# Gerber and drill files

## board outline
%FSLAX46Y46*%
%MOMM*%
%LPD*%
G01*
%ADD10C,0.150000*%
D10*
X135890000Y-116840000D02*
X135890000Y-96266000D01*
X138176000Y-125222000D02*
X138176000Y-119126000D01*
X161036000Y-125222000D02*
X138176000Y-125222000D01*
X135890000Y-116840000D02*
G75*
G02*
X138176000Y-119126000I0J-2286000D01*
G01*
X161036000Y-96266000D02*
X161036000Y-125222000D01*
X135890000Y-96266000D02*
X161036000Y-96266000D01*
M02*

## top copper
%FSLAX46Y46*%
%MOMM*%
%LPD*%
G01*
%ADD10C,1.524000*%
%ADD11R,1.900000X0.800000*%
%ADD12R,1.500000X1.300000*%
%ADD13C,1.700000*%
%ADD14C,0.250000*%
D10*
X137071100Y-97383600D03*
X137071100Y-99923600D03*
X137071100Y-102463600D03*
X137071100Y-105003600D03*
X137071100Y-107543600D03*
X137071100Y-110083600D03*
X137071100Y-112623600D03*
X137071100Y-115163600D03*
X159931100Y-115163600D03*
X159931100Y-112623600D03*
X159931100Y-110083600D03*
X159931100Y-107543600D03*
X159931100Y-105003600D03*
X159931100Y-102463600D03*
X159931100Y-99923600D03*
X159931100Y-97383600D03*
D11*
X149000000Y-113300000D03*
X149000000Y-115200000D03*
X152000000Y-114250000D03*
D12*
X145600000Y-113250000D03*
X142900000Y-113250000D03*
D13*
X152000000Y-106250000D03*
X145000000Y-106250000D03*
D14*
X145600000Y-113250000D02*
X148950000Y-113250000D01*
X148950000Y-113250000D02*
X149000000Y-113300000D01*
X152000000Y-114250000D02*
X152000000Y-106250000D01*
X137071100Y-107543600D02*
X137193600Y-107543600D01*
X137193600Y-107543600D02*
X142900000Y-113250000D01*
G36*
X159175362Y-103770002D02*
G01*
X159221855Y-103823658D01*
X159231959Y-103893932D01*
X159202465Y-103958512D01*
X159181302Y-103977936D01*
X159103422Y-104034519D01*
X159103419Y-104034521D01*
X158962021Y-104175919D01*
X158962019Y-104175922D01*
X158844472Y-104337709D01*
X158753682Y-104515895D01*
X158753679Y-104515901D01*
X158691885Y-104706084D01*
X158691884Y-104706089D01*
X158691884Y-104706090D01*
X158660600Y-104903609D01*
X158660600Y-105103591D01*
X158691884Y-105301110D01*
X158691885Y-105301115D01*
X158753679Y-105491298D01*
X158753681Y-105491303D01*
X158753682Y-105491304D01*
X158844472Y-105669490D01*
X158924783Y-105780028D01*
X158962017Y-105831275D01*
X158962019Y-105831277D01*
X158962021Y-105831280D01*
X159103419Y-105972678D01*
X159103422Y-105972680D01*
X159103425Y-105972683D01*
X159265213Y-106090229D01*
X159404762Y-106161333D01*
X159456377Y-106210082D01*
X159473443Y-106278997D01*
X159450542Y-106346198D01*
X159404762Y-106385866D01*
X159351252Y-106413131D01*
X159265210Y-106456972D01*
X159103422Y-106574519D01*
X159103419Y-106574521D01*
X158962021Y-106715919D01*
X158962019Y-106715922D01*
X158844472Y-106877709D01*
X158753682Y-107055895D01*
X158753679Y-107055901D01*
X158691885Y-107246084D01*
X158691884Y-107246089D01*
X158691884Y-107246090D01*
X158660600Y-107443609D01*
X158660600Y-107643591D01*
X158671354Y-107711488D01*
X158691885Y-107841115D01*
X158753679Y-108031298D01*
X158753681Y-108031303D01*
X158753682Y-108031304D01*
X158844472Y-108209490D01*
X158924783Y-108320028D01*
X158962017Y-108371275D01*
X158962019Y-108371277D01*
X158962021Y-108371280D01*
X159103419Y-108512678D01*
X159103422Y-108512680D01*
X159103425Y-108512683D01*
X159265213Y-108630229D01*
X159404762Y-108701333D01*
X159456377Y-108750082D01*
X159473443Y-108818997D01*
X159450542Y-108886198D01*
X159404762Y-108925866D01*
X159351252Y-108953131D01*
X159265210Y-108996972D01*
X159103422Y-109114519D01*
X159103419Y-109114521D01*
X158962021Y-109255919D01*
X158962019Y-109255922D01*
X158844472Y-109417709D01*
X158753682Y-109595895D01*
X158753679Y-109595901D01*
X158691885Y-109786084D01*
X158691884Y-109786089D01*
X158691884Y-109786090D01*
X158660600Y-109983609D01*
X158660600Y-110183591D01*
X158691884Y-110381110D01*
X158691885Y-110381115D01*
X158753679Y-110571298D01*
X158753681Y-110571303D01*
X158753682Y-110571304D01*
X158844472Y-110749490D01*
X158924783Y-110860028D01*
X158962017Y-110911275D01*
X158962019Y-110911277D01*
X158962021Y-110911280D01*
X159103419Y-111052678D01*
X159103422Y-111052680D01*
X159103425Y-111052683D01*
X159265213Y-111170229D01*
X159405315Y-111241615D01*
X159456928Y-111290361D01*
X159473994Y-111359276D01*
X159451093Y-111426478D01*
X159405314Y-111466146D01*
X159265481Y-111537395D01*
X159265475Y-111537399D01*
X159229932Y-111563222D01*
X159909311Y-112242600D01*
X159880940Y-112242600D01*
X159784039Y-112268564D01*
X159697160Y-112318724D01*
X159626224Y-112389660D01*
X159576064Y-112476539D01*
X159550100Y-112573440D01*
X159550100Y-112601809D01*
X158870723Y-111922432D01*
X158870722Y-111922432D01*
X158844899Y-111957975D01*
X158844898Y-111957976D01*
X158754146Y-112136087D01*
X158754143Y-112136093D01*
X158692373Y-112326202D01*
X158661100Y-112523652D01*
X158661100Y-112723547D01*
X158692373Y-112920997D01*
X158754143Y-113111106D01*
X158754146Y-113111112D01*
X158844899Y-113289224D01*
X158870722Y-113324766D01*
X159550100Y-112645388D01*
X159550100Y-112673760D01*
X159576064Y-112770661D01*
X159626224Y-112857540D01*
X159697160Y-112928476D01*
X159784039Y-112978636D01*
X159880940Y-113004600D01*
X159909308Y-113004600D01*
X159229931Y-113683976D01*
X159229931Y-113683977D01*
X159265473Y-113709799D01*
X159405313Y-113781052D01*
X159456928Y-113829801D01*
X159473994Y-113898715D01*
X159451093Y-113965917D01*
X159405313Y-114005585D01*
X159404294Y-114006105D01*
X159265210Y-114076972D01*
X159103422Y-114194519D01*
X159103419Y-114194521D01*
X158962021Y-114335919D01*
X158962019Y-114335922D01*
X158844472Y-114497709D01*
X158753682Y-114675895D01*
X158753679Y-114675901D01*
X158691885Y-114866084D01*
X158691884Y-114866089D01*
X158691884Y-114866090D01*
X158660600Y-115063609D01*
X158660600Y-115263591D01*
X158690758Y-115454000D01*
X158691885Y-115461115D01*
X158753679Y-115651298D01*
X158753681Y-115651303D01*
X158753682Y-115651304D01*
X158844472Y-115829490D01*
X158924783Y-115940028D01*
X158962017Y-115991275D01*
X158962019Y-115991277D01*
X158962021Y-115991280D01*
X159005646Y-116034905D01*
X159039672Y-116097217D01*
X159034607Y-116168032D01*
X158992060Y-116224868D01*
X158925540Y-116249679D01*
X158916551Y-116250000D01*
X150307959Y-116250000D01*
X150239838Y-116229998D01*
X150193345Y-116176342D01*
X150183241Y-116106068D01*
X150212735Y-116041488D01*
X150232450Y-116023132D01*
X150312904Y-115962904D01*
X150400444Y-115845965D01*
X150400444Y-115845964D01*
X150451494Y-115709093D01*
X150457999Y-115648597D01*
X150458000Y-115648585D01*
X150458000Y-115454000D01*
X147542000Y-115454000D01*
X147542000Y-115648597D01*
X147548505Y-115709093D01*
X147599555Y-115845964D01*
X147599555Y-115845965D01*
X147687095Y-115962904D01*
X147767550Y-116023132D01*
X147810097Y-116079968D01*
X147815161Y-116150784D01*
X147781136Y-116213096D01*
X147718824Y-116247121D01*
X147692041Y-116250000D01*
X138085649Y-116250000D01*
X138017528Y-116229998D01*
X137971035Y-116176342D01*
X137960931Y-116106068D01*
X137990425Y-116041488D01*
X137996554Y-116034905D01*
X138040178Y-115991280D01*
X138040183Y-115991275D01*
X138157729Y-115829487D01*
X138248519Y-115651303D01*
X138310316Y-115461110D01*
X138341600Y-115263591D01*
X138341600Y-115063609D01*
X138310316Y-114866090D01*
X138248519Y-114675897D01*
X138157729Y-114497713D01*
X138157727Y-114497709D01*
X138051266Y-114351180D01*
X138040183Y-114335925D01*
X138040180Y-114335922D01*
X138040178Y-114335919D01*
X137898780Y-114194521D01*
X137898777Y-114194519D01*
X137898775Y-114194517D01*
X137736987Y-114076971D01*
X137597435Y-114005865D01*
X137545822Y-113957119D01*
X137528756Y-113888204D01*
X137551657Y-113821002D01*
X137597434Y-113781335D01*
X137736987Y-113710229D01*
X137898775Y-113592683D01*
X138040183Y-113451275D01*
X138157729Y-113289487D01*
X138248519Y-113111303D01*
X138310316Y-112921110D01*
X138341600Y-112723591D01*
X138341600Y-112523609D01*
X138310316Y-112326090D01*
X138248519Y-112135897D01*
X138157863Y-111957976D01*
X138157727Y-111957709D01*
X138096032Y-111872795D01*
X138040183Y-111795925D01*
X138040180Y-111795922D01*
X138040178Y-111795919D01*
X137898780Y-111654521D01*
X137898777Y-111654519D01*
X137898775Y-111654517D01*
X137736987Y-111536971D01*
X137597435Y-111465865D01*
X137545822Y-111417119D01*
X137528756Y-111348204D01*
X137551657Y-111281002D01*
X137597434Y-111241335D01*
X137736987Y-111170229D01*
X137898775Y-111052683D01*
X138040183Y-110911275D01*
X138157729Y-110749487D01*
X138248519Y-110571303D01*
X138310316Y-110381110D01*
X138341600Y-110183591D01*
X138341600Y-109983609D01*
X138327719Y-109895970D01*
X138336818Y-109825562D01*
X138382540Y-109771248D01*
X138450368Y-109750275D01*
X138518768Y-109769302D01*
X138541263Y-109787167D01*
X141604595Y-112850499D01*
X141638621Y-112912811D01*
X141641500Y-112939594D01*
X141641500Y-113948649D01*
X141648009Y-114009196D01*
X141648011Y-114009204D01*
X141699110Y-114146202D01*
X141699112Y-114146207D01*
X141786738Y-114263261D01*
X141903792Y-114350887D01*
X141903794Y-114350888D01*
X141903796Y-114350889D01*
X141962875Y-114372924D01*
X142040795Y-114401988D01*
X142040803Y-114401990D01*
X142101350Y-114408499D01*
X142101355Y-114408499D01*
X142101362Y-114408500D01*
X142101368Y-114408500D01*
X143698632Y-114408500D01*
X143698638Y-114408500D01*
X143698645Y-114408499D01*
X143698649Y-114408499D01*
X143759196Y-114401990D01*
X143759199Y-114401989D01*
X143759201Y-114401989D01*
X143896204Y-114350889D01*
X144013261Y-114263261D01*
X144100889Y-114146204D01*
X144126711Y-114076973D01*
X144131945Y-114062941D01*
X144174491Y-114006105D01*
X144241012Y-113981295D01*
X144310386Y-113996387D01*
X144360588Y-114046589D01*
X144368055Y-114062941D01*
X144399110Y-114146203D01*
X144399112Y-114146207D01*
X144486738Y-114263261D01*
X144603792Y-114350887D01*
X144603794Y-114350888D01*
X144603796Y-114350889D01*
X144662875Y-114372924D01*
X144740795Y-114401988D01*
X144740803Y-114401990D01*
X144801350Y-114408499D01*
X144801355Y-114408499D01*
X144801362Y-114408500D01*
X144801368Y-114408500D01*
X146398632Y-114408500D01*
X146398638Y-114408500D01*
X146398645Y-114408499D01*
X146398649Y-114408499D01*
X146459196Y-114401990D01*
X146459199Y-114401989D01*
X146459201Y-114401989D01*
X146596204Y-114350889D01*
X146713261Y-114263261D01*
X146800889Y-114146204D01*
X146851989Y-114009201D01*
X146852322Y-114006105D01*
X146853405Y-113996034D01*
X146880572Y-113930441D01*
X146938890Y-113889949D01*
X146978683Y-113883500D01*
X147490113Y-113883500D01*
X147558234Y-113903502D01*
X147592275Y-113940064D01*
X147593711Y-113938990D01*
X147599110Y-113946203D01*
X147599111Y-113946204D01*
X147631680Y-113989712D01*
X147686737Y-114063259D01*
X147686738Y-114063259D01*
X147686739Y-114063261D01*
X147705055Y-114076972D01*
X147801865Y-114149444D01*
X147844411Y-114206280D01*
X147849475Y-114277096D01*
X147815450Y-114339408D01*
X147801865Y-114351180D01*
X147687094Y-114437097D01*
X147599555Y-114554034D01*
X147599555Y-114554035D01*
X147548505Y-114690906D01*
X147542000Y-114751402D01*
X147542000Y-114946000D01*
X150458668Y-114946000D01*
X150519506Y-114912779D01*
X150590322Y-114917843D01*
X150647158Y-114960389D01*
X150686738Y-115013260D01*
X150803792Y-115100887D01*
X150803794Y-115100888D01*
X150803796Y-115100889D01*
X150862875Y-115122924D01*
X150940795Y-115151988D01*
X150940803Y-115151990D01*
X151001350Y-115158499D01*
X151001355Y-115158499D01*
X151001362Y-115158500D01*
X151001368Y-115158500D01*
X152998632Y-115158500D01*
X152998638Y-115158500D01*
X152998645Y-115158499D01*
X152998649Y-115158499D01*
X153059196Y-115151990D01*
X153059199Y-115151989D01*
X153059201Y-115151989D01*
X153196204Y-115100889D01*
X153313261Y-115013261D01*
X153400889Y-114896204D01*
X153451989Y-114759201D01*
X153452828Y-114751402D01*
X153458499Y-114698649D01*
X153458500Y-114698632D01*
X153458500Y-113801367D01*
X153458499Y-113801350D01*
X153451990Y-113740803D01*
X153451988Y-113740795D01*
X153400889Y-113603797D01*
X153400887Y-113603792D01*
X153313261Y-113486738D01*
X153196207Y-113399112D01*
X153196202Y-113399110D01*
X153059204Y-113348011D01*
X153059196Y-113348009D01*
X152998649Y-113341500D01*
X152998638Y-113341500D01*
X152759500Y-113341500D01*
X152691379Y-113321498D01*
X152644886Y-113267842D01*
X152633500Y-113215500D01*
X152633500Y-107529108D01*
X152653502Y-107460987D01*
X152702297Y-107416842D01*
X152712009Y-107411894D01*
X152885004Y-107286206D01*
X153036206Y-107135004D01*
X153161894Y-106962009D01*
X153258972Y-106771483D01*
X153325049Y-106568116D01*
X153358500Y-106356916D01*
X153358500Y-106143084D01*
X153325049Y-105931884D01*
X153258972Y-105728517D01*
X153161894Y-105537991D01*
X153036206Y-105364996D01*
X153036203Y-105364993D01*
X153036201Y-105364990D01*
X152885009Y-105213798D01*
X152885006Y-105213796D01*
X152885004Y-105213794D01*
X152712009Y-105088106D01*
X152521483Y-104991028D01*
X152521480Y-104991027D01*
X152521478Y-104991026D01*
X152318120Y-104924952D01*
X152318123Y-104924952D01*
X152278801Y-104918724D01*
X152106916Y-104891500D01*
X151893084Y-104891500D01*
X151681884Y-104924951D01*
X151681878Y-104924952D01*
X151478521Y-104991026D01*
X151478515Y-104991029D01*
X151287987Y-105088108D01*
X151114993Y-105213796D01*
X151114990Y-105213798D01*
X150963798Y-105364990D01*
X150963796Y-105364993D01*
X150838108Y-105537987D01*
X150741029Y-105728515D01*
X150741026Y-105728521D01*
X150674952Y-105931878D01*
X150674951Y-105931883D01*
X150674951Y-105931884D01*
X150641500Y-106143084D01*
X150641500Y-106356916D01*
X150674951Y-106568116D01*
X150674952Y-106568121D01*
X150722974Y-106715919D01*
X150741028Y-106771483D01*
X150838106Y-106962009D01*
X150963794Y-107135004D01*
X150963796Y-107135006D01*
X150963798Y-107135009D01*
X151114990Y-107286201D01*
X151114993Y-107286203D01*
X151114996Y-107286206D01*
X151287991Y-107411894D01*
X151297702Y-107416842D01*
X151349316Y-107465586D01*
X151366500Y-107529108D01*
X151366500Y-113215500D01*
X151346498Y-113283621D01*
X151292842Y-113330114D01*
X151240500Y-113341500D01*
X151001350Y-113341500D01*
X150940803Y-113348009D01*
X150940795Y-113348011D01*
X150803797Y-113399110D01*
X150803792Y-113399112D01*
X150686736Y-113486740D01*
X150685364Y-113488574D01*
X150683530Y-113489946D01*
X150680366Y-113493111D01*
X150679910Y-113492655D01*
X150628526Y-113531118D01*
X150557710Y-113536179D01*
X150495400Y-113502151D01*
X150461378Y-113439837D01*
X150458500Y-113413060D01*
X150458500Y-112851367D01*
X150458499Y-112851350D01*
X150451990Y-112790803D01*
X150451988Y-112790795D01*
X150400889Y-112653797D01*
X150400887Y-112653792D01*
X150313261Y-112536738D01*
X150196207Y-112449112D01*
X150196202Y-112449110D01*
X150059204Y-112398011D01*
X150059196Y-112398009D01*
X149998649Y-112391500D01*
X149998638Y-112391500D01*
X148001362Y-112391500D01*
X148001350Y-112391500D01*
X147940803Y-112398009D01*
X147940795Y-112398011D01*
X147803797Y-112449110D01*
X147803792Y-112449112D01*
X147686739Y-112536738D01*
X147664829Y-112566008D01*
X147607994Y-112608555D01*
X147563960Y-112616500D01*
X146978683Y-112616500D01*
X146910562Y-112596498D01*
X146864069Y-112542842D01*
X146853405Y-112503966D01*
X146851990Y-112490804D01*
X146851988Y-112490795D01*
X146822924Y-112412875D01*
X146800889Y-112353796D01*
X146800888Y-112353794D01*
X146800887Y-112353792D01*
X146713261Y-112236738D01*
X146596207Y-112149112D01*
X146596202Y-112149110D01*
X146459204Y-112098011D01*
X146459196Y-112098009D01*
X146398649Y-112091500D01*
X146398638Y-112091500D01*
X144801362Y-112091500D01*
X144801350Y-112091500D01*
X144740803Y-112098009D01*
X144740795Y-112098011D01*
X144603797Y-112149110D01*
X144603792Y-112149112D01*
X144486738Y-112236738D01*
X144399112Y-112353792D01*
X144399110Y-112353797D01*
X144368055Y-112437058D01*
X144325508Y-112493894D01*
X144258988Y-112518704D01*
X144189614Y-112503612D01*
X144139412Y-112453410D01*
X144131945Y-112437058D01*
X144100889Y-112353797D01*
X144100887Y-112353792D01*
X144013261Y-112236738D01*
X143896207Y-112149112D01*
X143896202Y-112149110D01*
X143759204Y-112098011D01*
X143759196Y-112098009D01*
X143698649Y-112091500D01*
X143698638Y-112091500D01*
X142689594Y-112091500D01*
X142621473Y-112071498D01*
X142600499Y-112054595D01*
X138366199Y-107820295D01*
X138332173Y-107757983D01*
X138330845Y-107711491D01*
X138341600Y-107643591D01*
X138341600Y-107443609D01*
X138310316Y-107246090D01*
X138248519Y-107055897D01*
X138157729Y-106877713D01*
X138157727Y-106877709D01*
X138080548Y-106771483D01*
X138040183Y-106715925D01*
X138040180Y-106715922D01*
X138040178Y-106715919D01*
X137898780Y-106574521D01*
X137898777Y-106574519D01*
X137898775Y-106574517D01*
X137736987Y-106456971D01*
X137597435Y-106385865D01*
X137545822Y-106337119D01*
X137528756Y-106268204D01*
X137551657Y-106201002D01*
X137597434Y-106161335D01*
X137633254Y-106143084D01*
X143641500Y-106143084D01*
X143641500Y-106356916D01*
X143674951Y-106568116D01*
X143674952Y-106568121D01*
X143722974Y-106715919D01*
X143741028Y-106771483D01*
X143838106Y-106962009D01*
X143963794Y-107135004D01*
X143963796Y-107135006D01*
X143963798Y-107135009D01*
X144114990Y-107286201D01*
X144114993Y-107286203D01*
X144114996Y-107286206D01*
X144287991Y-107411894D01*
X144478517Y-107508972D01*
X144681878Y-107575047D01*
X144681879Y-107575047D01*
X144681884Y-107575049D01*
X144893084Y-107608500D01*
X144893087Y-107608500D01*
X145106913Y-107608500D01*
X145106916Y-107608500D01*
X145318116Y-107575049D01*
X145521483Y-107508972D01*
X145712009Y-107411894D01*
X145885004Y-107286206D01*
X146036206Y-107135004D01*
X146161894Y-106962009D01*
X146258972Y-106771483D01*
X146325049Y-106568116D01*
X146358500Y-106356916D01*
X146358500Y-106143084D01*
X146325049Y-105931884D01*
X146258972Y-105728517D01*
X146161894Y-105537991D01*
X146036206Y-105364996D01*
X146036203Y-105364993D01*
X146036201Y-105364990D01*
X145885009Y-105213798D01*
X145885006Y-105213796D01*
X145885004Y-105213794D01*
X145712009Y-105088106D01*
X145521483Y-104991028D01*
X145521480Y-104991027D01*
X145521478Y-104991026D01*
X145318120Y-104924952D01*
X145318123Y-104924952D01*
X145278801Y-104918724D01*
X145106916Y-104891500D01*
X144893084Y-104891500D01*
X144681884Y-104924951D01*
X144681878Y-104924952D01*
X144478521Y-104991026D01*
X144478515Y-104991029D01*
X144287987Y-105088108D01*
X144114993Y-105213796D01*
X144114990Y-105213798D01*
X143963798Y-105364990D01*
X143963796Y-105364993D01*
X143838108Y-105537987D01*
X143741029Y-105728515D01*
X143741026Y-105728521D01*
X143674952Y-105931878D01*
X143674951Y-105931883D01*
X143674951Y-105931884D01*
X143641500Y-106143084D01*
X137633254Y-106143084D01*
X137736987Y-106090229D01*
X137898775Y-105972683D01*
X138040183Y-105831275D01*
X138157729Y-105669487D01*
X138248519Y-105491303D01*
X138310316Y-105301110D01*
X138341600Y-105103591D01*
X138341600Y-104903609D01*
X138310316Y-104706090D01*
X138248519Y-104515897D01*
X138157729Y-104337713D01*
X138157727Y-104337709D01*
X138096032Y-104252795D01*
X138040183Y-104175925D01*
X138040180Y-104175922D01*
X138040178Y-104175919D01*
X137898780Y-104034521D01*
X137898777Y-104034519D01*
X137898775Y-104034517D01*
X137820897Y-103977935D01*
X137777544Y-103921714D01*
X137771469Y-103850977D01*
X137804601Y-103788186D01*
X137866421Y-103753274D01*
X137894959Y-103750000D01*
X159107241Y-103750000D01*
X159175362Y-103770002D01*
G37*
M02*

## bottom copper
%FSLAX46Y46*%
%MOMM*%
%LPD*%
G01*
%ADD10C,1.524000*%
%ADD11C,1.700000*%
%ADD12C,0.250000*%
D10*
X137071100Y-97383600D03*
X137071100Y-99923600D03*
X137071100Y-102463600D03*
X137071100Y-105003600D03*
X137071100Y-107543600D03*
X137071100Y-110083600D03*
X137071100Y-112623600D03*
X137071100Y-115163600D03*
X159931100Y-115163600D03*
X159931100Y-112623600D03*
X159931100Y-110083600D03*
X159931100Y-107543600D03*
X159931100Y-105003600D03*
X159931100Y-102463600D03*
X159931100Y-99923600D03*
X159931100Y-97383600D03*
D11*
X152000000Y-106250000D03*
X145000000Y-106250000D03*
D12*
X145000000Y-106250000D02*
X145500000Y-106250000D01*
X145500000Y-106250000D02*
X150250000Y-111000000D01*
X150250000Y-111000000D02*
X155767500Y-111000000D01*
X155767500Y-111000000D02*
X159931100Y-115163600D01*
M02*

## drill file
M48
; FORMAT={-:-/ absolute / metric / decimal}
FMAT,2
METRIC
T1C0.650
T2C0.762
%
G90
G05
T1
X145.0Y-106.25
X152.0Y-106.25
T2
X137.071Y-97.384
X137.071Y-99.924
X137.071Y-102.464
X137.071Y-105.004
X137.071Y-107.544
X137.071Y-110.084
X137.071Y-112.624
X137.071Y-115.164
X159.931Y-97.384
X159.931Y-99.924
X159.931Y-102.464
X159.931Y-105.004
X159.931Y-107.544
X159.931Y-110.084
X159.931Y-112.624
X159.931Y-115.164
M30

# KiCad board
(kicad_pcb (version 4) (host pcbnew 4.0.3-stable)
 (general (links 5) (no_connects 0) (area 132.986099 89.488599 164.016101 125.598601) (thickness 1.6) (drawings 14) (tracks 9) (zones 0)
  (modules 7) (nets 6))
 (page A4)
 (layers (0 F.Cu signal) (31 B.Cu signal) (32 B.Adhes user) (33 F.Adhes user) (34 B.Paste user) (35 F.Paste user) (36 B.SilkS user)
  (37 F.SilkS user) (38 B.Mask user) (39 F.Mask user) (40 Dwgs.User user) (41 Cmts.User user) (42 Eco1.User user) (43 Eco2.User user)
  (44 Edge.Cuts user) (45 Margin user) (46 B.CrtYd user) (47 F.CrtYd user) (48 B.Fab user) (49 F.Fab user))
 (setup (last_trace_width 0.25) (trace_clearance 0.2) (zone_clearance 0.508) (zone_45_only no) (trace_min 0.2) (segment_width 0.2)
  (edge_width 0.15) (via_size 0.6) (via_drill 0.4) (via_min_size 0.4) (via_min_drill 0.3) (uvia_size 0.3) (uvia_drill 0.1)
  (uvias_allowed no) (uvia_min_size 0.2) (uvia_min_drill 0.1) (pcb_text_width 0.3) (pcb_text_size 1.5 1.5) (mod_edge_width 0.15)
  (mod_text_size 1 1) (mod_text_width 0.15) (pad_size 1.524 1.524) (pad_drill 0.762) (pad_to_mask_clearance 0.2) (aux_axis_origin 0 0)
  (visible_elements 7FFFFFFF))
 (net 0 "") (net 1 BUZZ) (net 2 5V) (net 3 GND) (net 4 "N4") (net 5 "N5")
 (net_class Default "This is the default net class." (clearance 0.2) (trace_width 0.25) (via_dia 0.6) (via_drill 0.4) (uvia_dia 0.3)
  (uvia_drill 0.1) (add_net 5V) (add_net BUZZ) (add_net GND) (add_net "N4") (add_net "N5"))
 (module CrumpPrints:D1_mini (layer F.Cu) (at 148.5011 105.0036)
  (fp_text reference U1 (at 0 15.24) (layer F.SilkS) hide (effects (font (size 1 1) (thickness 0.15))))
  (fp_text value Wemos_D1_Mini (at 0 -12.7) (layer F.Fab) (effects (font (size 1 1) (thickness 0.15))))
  (pad 1 thru_hole circle (at -11.43 -7.62) (size 1.524 1.524) (drill 0.762) (layers *.Cu *.Mask))
  (pad 2 thru_hole circle (at -11.43 -5.08) (size 1.524 1.524) (drill 0.762) (layers *.Cu *.Mask))
  (pad 3 thru_hole circle (at -11.43 -2.54) (size 1.524 1.524) (drill 0.762) (layers *.Cu *.Mask))
  (pad 4 thru_hole circle (at -11.43 0) (size 1.524 1.524) (drill 0.762) (layers *.Cu *.Mask))
  (pad 5 thru_hole circle (at -11.43 2.54) (size 1.524 1.524) (drill 0.762) (layers *.Cu *.Mask) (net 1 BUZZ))
  (pad 6 thru_hole circle (at -11.43 5.08) (size 1.524 1.524) (drill 0.762) (layers *.Cu *.Mask))
  (pad 7 thru_hole circle (at -11.43 7.62) (size 1.524 1.524) (drill 0.762) (layers *.Cu *.Mask))
  (pad 8 thru_hole circle (at -11.43 10.16) (size 1.524 1.524) (drill 0.762) (layers *.Cu *.Mask))
  (pad 9 thru_hole circle (at 11.43 10.16) (size 1.524 1.524) (drill 0.762) (layers *.Cu *.Mask) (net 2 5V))
  (pad 10 thru_hole circle (at 11.43 7.62) (size 1.524 1.524) (drill 0.762) (layers *.Cu *.Mask) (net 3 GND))
  (pad 11 thru_hole circle (at 11.43 5.08) (size 1.524 1.524) (drill 0.762) (layers *.Cu *.Mask))
  (pad 12 thru_hole circle (at 11.43 2.54) (size 1.524 1.524) (drill 0.762) (layers *.Cu *.Mask))
  (pad 13 thru_hole circle (at 11.43 0) (size 1.524 1.524) (drill 0.762) (layers *.Cu *.Mask))
  (pad 14 thru_hole circle (at 11.43 -2.54) (size 1.524 1.524) (drill 0.762) (layers *.Cu *.Mask))
  (pad 15 thru_hole circle (at 11.43 -5.08) (size 1.524 1.524) (drill 0.762) (layers *.Cu *.Mask))
  (pad 16 thru_hole circle (at 11.43 -7.62) (size 1.524 1.524) (drill 0.762) (layers *.Cu *.Mask)))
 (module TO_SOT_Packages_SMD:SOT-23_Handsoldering (layer F.Cu) (at 150.5 114.25)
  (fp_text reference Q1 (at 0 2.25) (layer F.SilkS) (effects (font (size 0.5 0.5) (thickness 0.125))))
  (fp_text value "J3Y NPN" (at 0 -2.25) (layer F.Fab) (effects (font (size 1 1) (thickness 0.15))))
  (pad 1 smd rect (at -1.5 -0.95) (size 1.9 0.8) (layers F.Cu F.Paste F.Mask) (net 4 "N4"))
  (pad 2 smd rect (at -1.5 0.95) (size 1.9 0.8) (layers F.Cu F.Paste F.Mask) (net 3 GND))
  (pad 3 smd rect (at 1.5 0) (size 1.9 0.8) (layers F.Cu F.Paste F.Mask) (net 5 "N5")))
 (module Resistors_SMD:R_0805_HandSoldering (layer F.Cu) (at 144.25 113.25 180)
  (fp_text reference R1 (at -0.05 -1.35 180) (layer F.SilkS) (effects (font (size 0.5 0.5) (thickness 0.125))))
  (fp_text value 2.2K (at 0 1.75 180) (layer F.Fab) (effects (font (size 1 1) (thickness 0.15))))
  (pad 1 smd rect (at -1.35 0 180) (size 1.5 1.3) (layers F.Cu F.Paste F.Mask) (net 4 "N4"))
  (pad 2 smd rect (at 1.35 0 180) (size 1.5 1.3) (layers F.Cu F.Paste F.Mask) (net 1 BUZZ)))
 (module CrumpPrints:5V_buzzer (layer F.Cu) (at 148.5 106.25)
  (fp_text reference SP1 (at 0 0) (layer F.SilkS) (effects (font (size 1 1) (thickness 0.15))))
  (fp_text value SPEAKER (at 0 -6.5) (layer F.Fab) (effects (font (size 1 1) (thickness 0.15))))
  (pad 2 thru_hole circle (at 3.5 0) (size 1.7 1.7) (drill 0.65) (layers *.Cu *.Mask) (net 5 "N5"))
  (pad 1 thru_hole circle (at -3.5 0) (size 1.7 1.7) (drill 0.65) (layers *.Cu *.Mask) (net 2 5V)))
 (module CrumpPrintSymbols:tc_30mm (layer F.Cu) (at 154 98.75)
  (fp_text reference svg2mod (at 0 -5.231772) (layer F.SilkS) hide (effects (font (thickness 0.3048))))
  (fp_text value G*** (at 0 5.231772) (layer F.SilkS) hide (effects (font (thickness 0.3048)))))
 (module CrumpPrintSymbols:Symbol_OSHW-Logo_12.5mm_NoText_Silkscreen (layer B.Cu) (at 148.6 112.5 180)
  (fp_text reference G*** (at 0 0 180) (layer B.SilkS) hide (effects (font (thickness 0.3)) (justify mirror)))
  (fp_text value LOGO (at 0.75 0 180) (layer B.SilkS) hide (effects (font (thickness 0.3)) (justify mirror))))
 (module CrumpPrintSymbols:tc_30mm (layer B.Cu) (at 143.8 98.7 180)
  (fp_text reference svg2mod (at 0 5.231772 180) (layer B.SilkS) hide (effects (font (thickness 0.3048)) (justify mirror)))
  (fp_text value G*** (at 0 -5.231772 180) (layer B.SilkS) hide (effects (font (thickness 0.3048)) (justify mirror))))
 (gr_line (start 135.89 116.84) (end 135.89 96.266) (angle 90) (layer Edge.Cuts) (width 0.15))
 (gr_line (start 138.176 125.222) (end 138.176 119.126) (angle 90) (layer Edge.Cuts) (width 0.15))
 (gr_line (start 161.036 125.222) (end 138.176 125.222) (angle 90) (layer Edge.Cuts) (width 0.15))
 (gr_arc (start 135.89 119.126) (end 135.89 116.84) (angle 90) (layer Edge.Cuts) (width 0.15))
 (gr_line (start 161.036 96.266) (end 161.036 125.222) (angle 90) (layer Edge.Cuts) (width 0.15))
 (gr_line (start 135.89 96.266) (end 161.036 96.266) (angle 90) (layer Edge.Cuts) (width 0.15))
 (segment (start 145.6 113.25) (end 148.95 113.25) (width 0.25) (layer F.Cu) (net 4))
 (segment (start 148.95 113.25) (end 149 113.3) (width 0.25) (layer F.Cu) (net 4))
 (segment (start 152 114.25) (end 152 106.25) (width 0.25) (layer F.Cu) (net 5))
 (segment (start 137.0711 107.5436) (end 137.1936 107.5436) (width 0.25) (layer F.Cu) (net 1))
 (segment (start 137.1936 107.5436) (end 142.9 113.25) (width 0.25) (layer F.Cu) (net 1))
 (segment (start 145 106.25) (end 145.5 106.25) (width 0.25) (layer B.Cu) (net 2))
 (segment (start 145.5 106.25) (end 150.25 111) (width 0.25) (layer B.Cu) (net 2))
 (segment (start 150.25 111) (end 155.7675 111) (width 0.25) (layer B.Cu) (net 2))
 (segment (start 155.7675 111) (end 159.9311 115.1636) (width 0.25) (layer B.Cu) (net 2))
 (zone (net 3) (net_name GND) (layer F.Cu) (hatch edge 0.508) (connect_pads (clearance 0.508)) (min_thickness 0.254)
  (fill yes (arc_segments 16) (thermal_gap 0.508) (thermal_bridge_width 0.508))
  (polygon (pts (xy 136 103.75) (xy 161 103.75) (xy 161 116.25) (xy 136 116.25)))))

